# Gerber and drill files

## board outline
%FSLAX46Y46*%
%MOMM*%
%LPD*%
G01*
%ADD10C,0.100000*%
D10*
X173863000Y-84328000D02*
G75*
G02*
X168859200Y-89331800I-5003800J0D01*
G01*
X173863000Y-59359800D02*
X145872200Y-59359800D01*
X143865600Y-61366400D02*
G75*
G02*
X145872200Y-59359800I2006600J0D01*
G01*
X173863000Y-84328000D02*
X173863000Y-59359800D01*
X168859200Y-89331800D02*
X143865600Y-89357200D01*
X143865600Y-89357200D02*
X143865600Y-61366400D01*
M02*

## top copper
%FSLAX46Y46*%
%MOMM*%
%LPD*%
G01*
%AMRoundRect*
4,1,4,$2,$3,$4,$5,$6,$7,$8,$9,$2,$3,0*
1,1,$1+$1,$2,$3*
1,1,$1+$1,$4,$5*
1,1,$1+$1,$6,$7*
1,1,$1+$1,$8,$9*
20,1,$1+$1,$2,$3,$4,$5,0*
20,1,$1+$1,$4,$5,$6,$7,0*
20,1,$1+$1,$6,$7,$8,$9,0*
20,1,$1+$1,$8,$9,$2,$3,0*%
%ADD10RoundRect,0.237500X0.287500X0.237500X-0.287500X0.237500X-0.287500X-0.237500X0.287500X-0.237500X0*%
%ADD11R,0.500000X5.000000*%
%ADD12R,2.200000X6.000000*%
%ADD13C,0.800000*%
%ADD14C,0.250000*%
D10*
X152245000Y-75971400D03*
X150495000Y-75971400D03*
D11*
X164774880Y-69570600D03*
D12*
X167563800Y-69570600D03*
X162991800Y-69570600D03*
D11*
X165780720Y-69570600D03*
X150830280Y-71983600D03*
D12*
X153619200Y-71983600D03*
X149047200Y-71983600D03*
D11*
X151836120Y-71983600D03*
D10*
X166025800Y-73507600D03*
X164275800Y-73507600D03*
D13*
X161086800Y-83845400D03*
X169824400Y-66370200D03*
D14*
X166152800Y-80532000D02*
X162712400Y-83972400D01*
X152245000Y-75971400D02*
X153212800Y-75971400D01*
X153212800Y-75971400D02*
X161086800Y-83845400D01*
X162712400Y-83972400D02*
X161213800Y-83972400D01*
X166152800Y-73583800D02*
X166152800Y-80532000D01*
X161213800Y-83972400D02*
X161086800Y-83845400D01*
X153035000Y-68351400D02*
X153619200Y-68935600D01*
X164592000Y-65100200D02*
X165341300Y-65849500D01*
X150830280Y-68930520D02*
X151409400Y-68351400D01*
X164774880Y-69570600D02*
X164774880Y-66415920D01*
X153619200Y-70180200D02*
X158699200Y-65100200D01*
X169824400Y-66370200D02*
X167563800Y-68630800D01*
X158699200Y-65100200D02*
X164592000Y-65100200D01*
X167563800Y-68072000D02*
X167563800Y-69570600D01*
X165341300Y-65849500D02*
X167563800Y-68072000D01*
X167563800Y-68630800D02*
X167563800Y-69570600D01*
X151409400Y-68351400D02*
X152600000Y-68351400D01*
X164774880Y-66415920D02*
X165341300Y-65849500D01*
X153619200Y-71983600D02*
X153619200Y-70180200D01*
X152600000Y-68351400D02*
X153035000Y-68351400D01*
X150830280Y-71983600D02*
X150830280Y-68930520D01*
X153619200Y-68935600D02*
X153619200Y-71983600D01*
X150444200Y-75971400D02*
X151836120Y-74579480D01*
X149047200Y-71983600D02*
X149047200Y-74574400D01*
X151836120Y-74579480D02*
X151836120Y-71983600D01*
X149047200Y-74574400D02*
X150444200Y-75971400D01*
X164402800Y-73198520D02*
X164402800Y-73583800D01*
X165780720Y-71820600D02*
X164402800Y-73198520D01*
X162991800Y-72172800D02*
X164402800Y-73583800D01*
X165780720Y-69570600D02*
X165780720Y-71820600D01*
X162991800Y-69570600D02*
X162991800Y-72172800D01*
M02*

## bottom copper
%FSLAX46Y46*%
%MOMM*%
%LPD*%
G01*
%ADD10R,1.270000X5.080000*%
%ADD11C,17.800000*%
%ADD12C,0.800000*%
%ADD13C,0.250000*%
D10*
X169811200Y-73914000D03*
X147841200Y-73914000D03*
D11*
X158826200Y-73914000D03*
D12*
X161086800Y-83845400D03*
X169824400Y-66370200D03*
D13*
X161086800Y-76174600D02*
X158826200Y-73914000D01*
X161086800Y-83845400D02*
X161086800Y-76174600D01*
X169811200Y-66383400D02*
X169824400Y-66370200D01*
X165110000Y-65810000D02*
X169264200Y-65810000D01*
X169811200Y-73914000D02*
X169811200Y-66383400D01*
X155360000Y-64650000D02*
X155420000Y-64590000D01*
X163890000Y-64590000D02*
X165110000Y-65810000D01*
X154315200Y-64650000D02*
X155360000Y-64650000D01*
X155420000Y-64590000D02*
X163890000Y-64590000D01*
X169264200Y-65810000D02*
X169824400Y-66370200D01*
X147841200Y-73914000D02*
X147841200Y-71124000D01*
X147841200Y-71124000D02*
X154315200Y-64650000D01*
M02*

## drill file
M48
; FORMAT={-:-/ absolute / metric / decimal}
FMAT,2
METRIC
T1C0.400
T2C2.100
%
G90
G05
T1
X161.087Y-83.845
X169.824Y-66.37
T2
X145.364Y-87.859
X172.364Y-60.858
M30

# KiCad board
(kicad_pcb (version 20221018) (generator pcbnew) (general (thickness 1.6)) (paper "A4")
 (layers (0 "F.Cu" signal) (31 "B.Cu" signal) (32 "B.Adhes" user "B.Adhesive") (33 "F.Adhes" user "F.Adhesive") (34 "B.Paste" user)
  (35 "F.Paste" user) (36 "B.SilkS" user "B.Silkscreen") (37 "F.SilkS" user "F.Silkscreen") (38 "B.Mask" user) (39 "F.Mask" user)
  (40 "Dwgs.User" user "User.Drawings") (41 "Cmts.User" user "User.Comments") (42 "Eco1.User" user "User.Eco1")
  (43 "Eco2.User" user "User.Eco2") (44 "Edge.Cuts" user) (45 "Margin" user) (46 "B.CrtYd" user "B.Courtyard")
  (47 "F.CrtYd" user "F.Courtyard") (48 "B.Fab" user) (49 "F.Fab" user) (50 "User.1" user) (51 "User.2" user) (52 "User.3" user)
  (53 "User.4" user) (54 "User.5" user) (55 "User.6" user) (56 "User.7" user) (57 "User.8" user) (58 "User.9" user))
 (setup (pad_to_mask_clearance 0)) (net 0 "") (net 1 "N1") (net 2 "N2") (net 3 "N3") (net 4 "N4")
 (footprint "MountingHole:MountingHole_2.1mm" (layer "F.Cu") (at 145.3642 87.8586)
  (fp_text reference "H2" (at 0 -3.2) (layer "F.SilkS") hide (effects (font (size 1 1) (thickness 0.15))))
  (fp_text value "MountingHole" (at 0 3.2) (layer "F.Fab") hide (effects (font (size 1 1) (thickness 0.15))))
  (pad "" np_thru_hole circle (at 0 0) (size 2.1 2.1) (drill 2.1) (layers "*.Cu" "*.Mask")))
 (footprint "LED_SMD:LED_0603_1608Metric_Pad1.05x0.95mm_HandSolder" (layer "F.Cu") (at 151.37 75.9714 180)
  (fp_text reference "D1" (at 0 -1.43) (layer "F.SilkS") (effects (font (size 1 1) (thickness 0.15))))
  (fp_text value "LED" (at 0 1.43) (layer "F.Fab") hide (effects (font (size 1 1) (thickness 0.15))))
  (pad "1" smd roundrect (at -0.875 0 180) (size 1.05 0.95) (layers "F.Cu" "F.Paste" "F.Mask") (roundrect_rratio 0.25) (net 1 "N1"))
  (pad "2" smd roundrect (at 0.875 0 180) (size 1.05 0.95) (layers "F.Cu" "F.Paste" "F.Mask") (roundrect_rratio 0.25) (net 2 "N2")))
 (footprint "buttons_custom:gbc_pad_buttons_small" (layer "F.Cu") (at 165.2778 69.5706)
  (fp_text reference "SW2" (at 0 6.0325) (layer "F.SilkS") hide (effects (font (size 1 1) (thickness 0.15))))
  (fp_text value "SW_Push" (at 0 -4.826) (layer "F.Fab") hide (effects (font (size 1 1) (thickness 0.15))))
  (pad "1" smd rect (at -0.50292 0 90) (size 5 0.5) (layers "F.Cu" "F.Paste" "F.Mask") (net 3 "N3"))
  (pad "1" smd rect (at 2.286 0) (size 2.2 6) (layers "F.Cu" "F.Paste" "F.Mask") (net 3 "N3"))
  (pad "2" smd rect (at -2.286 0) (size 2.2 6) (layers "F.Cu" "F.Paste" "F.Mask") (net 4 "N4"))
  (pad "2" smd rect (at 0.50292 0 90) (size 5 0.5) (layers "F.Cu" "F.Paste" "F.Mask") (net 4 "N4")))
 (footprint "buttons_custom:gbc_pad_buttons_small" (layer "F.Cu") (at 151.3332 71.9836)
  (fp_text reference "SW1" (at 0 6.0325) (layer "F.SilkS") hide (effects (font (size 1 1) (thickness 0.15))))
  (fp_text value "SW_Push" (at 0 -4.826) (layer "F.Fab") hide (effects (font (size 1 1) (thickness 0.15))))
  (pad "1" smd rect (at -0.50292 0 90) (size 5 0.5) (layers "F.Cu" "F.Paste" "F.Mask") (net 3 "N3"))
  (pad "1" smd rect (at 2.286 0) (size 2.2 6) (layers "F.Cu" "F.Paste" "F.Mask") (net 3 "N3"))
  (pad "2" smd rect (at -2.286 0) (size 2.2 6) (layers "F.Cu" "F.Paste" "F.Mask") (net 2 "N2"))
  (pad "2" smd rect (at 0.50292 0 90) (size 5 0.5) (layers "F.Cu" "F.Paste" "F.Mask") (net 2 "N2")))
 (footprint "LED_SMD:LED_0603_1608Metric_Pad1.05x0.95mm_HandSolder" (layer "F.Cu") (at 165.1508 73.5076 180)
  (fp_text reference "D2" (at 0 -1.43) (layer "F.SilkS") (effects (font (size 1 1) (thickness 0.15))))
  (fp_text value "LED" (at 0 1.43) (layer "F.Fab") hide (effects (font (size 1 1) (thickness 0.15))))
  (pad "1" smd roundrect (at -0.875 0 180) (size 1.05 0.95) (layers "F.Cu" "F.Paste" "F.Mask") (roundrect_rratio 0.25) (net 1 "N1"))
  (pad "2" smd roundrect (at 0.875 0 180) (size 1.05 0.95) (layers "F.Cu" "F.Paste" "F.Mask") (roundrect_rratio 0.25) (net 4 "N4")))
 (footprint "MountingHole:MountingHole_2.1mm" (layer "F.Cu") (at 172.3644 60.8584)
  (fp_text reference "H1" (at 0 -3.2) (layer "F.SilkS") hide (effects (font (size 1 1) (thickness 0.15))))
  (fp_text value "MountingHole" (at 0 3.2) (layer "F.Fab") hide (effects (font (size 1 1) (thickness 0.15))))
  (pad "" np_thru_hole circle (at 0 0) (size 2.1 2.1) (drill 2.1) (layers "*.Cu" "*.Mask")))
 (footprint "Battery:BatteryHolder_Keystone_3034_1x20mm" (layer "B.Cu") (at 158.8262 73.914 180)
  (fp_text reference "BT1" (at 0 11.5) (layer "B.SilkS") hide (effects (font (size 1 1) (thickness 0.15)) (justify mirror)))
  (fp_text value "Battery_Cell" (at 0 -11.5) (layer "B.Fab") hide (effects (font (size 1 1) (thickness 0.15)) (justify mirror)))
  (pad "1" smd rect (at -10.985 0 180) (size 1.27 5.08) (layers "B.Cu" "B.Paste" "B.Mask") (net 3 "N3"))
  (pad "1" smd rect (at 10.985 0 180) (size 1.27 5.08) (layers "B.Cu" "B.Paste" "B.Mask") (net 3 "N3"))
  (pad "2" smd circle (at 0 0 180) (size 17.8 17.8) (layers "B.Cu" "B.Mask") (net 1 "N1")))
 (gr_arc (start 173.863 84.328) (mid 172.397421 87.866221) (end 168.8592 89.3318) (stroke (width 0.1) (type default)) (layer "Edge.Cuts"))
 (gr_line (start 173.863 59.3598) (end 145.8722 59.3598) (stroke (width 0.1) (type default)) (layer "Edge.Cuts"))
 (gr_arc (start 143.8656 61.3664) (mid 144.45332 59.94752) (end 145.8722 59.3598) (stroke (width 0.1) (type default)) (layer "Edge.Cuts"))
 (gr_line (start 173.863 84.328) (end 173.863 59.3598) (stroke (width 0.1) (type default)) (layer "Edge.Cuts"))
 (gr_line (start 168.8592 89.3318) (end 143.8656 89.3572) (stroke (width 0.1) (type default)) (layer "Edge.Cuts"))
 (gr_line (start 143.8656 89.3572) (end 143.8656 61.3664) (stroke (width 0.1) (type default)) (layer "Edge.Cuts"))
 (segment (start 166.1528 80.532) (end 162.7124 83.9724) (width 0.25) (layer "F.Cu") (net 1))
 (segment (start 152.245 75.9714) (end 153.2128 75.9714) (width 0.25) (layer "F.Cu") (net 1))
 (segment (start 153.2128 75.9714) (end 161.0868 83.8454) (width 0.25) (layer "F.Cu") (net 1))
 (segment (start 162.7124 83.9724) (end 161.2138 83.9724) (width 0.25) (layer "F.Cu") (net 1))
 (segment (start 166.1528 73.5838) (end 166.1528 80.532) (width 0.25) (layer "F.Cu") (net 1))
 (segment (start 161.2138 83.9724) (end 161.0868 83.8454) (width 0.25) (layer "F.Cu") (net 1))
 (via (at 161.0868 83.8454) (size 0.8) (drill 0.4) (layers "F.Cu" "B.Cu") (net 1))
 (segment (start 161.0868 76.1746) (end 158.8262 73.914) (width 0.25) (layer "B.Cu") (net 1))
 (segment (start 161.0868 83.8454) (end 161.0868 76.1746) (width 0.25) (layer "B.Cu") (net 1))
 (segment (start 153.035 68.3514) (end 153.6192 68.9356) (width 0.25) (layer "F.Cu") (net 3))
 (segment (start 164.592 65.1002) (end 165.3413 65.8495) (width 0.25) (layer "F.Cu") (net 3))
 (segment (start 150.83028 68.93052) (end 151.4094 68.3514) (width 0.25) (layer "F.Cu") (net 3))
 (segment (start 164.77488 69.5706) (end 164.77488 66.41592) (width 0.25) (layer "F.Cu") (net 3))
 (segment (start 153.6192 70.1802) (end 158.6992 65.1002) (width 0.25) (layer "F.Cu") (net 3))
 (segment (start 169.8244 66.3702) (end 167.5638 68.6308) (width 0.25) (layer "F.Cu") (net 3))
 (segment (start 158.6992 65.1002) (end 164.592 65.1002) (width 0.25) (layer "F.Cu") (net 3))
 (segment (start 167.5638 68.072) (end 167.5638 69.5706) (width 0.25) (layer "F.Cu") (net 3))
 (segment (start 165.3413 65.8495) (end 167.5638 68.072) (width 0.25) (layer "F.Cu") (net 3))
 (segment (start 167.5638 68.6308) (end 167.5638 69.5706) (width 0.25) (layer "F.Cu") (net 3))
 (segment (start 151.4094 68.3514) (end 152.6 68.3514) (width 0.25) (layer "F.Cu") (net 3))
 (segment (start 164.77488 66.41592) (end 165.3413 65.8495) (width 0.25) (layer "F.Cu") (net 3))
 (segment (start 153.6192 71.9836) (end 153.6192 70.1802) (width 0.25) (layer "F.Cu") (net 3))
 (segment (start 152.6 68.3514) (end 153.035 68.3514) (width 0.25) (layer "F.Cu") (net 3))
 (segment (start 150.83028 71.9836) (end 150.83028 68.93052) (width 0.25) (layer "F.Cu") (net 3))
 (segment (start 153.6192 68.9356) (end 153.6192 71.9836) (width 0.25) (layer "F.Cu") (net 3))
 (via (at 169.8244 66.3702) (size 0.8) (drill 0.4) (layers "F.Cu" "B.Cu") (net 3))
 (segment (start 169.8112 66.3834) (end 169.8244 66.3702) (width 0.25) (layer "B.Cu") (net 3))
 (segment (start 165.11 65.81) (end 169.2642 65.81) (width 0.25) (layer "B.Cu") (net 3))
 (segment (start 169.8112 73.914) (end 169.8112 66.3834) (width 0.25) (layer "B.Cu") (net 3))
 (segment (start 155.36 64.65) (end 155.42 64.59) (width 0.25) (layer "B.Cu") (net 3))
 (segment (start 163.89 64.59) (end 165.11 65.81) (width 0.25) (layer "B.Cu") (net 3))
 (segment (start 154.3152 64.65) (end 155.36 64.65) (width 0.25) (layer "B.Cu") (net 3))
 (segment (start 155.42 64.59) (end 163.89 64.59) (width 0.25) (layer "B.Cu") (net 3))
 (segment (start 169.2642 65.81) (end 169.8244 66.3702) (width 0.25) (layer "B.Cu") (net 3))
 (segment (start 147.8412 73.914) (end 147.8412 71.124) (width 0.25) (layer "B.Cu") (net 3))
 (segment (start 147.8412 71.124) (end 154.3152 64.65) (width 0.25) (layer "B.Cu") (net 3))
 (segment (start 150.4442 75.9714) (end 151.83612 74.57948) (width 0.25) (layer "F.Cu") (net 2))
 (segment (start 149.0472 71.9836) (end 149.0472 74.5744) (width 0.25) (layer "F.Cu") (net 2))
 (segment (start 151.83612 74.57948) (end 151.83612 71.9836) (width 0.25) (layer "F.Cu") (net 2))
 (segment (start 149.0472 74.5744) (end 150.4442 75.9714) (width 0.25) (layer "F.Cu") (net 2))
 (segment (start 164.4028 73.19852) (end 164.4028 73.5838) (width 0.25) (layer "F.Cu") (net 4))
 (segment (start 165.78072 71.8206) (end 164.4028 73.19852) (width 0.25) (layer "F.Cu") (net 4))
 (segment (start 162.9918 72.1728) (end 164.4028 73.5838) (width 0.25) (layer "F.Cu") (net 4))
 (segment (start 165.78072 69.5706) (end 165.78072 71.8206) (width 0.25) (layer "F.Cu") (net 4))
 (segment (start 162.9918 69.5706) (end 162.9918 72.1728) (width 0.25) (layer "F.Cu") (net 4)))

